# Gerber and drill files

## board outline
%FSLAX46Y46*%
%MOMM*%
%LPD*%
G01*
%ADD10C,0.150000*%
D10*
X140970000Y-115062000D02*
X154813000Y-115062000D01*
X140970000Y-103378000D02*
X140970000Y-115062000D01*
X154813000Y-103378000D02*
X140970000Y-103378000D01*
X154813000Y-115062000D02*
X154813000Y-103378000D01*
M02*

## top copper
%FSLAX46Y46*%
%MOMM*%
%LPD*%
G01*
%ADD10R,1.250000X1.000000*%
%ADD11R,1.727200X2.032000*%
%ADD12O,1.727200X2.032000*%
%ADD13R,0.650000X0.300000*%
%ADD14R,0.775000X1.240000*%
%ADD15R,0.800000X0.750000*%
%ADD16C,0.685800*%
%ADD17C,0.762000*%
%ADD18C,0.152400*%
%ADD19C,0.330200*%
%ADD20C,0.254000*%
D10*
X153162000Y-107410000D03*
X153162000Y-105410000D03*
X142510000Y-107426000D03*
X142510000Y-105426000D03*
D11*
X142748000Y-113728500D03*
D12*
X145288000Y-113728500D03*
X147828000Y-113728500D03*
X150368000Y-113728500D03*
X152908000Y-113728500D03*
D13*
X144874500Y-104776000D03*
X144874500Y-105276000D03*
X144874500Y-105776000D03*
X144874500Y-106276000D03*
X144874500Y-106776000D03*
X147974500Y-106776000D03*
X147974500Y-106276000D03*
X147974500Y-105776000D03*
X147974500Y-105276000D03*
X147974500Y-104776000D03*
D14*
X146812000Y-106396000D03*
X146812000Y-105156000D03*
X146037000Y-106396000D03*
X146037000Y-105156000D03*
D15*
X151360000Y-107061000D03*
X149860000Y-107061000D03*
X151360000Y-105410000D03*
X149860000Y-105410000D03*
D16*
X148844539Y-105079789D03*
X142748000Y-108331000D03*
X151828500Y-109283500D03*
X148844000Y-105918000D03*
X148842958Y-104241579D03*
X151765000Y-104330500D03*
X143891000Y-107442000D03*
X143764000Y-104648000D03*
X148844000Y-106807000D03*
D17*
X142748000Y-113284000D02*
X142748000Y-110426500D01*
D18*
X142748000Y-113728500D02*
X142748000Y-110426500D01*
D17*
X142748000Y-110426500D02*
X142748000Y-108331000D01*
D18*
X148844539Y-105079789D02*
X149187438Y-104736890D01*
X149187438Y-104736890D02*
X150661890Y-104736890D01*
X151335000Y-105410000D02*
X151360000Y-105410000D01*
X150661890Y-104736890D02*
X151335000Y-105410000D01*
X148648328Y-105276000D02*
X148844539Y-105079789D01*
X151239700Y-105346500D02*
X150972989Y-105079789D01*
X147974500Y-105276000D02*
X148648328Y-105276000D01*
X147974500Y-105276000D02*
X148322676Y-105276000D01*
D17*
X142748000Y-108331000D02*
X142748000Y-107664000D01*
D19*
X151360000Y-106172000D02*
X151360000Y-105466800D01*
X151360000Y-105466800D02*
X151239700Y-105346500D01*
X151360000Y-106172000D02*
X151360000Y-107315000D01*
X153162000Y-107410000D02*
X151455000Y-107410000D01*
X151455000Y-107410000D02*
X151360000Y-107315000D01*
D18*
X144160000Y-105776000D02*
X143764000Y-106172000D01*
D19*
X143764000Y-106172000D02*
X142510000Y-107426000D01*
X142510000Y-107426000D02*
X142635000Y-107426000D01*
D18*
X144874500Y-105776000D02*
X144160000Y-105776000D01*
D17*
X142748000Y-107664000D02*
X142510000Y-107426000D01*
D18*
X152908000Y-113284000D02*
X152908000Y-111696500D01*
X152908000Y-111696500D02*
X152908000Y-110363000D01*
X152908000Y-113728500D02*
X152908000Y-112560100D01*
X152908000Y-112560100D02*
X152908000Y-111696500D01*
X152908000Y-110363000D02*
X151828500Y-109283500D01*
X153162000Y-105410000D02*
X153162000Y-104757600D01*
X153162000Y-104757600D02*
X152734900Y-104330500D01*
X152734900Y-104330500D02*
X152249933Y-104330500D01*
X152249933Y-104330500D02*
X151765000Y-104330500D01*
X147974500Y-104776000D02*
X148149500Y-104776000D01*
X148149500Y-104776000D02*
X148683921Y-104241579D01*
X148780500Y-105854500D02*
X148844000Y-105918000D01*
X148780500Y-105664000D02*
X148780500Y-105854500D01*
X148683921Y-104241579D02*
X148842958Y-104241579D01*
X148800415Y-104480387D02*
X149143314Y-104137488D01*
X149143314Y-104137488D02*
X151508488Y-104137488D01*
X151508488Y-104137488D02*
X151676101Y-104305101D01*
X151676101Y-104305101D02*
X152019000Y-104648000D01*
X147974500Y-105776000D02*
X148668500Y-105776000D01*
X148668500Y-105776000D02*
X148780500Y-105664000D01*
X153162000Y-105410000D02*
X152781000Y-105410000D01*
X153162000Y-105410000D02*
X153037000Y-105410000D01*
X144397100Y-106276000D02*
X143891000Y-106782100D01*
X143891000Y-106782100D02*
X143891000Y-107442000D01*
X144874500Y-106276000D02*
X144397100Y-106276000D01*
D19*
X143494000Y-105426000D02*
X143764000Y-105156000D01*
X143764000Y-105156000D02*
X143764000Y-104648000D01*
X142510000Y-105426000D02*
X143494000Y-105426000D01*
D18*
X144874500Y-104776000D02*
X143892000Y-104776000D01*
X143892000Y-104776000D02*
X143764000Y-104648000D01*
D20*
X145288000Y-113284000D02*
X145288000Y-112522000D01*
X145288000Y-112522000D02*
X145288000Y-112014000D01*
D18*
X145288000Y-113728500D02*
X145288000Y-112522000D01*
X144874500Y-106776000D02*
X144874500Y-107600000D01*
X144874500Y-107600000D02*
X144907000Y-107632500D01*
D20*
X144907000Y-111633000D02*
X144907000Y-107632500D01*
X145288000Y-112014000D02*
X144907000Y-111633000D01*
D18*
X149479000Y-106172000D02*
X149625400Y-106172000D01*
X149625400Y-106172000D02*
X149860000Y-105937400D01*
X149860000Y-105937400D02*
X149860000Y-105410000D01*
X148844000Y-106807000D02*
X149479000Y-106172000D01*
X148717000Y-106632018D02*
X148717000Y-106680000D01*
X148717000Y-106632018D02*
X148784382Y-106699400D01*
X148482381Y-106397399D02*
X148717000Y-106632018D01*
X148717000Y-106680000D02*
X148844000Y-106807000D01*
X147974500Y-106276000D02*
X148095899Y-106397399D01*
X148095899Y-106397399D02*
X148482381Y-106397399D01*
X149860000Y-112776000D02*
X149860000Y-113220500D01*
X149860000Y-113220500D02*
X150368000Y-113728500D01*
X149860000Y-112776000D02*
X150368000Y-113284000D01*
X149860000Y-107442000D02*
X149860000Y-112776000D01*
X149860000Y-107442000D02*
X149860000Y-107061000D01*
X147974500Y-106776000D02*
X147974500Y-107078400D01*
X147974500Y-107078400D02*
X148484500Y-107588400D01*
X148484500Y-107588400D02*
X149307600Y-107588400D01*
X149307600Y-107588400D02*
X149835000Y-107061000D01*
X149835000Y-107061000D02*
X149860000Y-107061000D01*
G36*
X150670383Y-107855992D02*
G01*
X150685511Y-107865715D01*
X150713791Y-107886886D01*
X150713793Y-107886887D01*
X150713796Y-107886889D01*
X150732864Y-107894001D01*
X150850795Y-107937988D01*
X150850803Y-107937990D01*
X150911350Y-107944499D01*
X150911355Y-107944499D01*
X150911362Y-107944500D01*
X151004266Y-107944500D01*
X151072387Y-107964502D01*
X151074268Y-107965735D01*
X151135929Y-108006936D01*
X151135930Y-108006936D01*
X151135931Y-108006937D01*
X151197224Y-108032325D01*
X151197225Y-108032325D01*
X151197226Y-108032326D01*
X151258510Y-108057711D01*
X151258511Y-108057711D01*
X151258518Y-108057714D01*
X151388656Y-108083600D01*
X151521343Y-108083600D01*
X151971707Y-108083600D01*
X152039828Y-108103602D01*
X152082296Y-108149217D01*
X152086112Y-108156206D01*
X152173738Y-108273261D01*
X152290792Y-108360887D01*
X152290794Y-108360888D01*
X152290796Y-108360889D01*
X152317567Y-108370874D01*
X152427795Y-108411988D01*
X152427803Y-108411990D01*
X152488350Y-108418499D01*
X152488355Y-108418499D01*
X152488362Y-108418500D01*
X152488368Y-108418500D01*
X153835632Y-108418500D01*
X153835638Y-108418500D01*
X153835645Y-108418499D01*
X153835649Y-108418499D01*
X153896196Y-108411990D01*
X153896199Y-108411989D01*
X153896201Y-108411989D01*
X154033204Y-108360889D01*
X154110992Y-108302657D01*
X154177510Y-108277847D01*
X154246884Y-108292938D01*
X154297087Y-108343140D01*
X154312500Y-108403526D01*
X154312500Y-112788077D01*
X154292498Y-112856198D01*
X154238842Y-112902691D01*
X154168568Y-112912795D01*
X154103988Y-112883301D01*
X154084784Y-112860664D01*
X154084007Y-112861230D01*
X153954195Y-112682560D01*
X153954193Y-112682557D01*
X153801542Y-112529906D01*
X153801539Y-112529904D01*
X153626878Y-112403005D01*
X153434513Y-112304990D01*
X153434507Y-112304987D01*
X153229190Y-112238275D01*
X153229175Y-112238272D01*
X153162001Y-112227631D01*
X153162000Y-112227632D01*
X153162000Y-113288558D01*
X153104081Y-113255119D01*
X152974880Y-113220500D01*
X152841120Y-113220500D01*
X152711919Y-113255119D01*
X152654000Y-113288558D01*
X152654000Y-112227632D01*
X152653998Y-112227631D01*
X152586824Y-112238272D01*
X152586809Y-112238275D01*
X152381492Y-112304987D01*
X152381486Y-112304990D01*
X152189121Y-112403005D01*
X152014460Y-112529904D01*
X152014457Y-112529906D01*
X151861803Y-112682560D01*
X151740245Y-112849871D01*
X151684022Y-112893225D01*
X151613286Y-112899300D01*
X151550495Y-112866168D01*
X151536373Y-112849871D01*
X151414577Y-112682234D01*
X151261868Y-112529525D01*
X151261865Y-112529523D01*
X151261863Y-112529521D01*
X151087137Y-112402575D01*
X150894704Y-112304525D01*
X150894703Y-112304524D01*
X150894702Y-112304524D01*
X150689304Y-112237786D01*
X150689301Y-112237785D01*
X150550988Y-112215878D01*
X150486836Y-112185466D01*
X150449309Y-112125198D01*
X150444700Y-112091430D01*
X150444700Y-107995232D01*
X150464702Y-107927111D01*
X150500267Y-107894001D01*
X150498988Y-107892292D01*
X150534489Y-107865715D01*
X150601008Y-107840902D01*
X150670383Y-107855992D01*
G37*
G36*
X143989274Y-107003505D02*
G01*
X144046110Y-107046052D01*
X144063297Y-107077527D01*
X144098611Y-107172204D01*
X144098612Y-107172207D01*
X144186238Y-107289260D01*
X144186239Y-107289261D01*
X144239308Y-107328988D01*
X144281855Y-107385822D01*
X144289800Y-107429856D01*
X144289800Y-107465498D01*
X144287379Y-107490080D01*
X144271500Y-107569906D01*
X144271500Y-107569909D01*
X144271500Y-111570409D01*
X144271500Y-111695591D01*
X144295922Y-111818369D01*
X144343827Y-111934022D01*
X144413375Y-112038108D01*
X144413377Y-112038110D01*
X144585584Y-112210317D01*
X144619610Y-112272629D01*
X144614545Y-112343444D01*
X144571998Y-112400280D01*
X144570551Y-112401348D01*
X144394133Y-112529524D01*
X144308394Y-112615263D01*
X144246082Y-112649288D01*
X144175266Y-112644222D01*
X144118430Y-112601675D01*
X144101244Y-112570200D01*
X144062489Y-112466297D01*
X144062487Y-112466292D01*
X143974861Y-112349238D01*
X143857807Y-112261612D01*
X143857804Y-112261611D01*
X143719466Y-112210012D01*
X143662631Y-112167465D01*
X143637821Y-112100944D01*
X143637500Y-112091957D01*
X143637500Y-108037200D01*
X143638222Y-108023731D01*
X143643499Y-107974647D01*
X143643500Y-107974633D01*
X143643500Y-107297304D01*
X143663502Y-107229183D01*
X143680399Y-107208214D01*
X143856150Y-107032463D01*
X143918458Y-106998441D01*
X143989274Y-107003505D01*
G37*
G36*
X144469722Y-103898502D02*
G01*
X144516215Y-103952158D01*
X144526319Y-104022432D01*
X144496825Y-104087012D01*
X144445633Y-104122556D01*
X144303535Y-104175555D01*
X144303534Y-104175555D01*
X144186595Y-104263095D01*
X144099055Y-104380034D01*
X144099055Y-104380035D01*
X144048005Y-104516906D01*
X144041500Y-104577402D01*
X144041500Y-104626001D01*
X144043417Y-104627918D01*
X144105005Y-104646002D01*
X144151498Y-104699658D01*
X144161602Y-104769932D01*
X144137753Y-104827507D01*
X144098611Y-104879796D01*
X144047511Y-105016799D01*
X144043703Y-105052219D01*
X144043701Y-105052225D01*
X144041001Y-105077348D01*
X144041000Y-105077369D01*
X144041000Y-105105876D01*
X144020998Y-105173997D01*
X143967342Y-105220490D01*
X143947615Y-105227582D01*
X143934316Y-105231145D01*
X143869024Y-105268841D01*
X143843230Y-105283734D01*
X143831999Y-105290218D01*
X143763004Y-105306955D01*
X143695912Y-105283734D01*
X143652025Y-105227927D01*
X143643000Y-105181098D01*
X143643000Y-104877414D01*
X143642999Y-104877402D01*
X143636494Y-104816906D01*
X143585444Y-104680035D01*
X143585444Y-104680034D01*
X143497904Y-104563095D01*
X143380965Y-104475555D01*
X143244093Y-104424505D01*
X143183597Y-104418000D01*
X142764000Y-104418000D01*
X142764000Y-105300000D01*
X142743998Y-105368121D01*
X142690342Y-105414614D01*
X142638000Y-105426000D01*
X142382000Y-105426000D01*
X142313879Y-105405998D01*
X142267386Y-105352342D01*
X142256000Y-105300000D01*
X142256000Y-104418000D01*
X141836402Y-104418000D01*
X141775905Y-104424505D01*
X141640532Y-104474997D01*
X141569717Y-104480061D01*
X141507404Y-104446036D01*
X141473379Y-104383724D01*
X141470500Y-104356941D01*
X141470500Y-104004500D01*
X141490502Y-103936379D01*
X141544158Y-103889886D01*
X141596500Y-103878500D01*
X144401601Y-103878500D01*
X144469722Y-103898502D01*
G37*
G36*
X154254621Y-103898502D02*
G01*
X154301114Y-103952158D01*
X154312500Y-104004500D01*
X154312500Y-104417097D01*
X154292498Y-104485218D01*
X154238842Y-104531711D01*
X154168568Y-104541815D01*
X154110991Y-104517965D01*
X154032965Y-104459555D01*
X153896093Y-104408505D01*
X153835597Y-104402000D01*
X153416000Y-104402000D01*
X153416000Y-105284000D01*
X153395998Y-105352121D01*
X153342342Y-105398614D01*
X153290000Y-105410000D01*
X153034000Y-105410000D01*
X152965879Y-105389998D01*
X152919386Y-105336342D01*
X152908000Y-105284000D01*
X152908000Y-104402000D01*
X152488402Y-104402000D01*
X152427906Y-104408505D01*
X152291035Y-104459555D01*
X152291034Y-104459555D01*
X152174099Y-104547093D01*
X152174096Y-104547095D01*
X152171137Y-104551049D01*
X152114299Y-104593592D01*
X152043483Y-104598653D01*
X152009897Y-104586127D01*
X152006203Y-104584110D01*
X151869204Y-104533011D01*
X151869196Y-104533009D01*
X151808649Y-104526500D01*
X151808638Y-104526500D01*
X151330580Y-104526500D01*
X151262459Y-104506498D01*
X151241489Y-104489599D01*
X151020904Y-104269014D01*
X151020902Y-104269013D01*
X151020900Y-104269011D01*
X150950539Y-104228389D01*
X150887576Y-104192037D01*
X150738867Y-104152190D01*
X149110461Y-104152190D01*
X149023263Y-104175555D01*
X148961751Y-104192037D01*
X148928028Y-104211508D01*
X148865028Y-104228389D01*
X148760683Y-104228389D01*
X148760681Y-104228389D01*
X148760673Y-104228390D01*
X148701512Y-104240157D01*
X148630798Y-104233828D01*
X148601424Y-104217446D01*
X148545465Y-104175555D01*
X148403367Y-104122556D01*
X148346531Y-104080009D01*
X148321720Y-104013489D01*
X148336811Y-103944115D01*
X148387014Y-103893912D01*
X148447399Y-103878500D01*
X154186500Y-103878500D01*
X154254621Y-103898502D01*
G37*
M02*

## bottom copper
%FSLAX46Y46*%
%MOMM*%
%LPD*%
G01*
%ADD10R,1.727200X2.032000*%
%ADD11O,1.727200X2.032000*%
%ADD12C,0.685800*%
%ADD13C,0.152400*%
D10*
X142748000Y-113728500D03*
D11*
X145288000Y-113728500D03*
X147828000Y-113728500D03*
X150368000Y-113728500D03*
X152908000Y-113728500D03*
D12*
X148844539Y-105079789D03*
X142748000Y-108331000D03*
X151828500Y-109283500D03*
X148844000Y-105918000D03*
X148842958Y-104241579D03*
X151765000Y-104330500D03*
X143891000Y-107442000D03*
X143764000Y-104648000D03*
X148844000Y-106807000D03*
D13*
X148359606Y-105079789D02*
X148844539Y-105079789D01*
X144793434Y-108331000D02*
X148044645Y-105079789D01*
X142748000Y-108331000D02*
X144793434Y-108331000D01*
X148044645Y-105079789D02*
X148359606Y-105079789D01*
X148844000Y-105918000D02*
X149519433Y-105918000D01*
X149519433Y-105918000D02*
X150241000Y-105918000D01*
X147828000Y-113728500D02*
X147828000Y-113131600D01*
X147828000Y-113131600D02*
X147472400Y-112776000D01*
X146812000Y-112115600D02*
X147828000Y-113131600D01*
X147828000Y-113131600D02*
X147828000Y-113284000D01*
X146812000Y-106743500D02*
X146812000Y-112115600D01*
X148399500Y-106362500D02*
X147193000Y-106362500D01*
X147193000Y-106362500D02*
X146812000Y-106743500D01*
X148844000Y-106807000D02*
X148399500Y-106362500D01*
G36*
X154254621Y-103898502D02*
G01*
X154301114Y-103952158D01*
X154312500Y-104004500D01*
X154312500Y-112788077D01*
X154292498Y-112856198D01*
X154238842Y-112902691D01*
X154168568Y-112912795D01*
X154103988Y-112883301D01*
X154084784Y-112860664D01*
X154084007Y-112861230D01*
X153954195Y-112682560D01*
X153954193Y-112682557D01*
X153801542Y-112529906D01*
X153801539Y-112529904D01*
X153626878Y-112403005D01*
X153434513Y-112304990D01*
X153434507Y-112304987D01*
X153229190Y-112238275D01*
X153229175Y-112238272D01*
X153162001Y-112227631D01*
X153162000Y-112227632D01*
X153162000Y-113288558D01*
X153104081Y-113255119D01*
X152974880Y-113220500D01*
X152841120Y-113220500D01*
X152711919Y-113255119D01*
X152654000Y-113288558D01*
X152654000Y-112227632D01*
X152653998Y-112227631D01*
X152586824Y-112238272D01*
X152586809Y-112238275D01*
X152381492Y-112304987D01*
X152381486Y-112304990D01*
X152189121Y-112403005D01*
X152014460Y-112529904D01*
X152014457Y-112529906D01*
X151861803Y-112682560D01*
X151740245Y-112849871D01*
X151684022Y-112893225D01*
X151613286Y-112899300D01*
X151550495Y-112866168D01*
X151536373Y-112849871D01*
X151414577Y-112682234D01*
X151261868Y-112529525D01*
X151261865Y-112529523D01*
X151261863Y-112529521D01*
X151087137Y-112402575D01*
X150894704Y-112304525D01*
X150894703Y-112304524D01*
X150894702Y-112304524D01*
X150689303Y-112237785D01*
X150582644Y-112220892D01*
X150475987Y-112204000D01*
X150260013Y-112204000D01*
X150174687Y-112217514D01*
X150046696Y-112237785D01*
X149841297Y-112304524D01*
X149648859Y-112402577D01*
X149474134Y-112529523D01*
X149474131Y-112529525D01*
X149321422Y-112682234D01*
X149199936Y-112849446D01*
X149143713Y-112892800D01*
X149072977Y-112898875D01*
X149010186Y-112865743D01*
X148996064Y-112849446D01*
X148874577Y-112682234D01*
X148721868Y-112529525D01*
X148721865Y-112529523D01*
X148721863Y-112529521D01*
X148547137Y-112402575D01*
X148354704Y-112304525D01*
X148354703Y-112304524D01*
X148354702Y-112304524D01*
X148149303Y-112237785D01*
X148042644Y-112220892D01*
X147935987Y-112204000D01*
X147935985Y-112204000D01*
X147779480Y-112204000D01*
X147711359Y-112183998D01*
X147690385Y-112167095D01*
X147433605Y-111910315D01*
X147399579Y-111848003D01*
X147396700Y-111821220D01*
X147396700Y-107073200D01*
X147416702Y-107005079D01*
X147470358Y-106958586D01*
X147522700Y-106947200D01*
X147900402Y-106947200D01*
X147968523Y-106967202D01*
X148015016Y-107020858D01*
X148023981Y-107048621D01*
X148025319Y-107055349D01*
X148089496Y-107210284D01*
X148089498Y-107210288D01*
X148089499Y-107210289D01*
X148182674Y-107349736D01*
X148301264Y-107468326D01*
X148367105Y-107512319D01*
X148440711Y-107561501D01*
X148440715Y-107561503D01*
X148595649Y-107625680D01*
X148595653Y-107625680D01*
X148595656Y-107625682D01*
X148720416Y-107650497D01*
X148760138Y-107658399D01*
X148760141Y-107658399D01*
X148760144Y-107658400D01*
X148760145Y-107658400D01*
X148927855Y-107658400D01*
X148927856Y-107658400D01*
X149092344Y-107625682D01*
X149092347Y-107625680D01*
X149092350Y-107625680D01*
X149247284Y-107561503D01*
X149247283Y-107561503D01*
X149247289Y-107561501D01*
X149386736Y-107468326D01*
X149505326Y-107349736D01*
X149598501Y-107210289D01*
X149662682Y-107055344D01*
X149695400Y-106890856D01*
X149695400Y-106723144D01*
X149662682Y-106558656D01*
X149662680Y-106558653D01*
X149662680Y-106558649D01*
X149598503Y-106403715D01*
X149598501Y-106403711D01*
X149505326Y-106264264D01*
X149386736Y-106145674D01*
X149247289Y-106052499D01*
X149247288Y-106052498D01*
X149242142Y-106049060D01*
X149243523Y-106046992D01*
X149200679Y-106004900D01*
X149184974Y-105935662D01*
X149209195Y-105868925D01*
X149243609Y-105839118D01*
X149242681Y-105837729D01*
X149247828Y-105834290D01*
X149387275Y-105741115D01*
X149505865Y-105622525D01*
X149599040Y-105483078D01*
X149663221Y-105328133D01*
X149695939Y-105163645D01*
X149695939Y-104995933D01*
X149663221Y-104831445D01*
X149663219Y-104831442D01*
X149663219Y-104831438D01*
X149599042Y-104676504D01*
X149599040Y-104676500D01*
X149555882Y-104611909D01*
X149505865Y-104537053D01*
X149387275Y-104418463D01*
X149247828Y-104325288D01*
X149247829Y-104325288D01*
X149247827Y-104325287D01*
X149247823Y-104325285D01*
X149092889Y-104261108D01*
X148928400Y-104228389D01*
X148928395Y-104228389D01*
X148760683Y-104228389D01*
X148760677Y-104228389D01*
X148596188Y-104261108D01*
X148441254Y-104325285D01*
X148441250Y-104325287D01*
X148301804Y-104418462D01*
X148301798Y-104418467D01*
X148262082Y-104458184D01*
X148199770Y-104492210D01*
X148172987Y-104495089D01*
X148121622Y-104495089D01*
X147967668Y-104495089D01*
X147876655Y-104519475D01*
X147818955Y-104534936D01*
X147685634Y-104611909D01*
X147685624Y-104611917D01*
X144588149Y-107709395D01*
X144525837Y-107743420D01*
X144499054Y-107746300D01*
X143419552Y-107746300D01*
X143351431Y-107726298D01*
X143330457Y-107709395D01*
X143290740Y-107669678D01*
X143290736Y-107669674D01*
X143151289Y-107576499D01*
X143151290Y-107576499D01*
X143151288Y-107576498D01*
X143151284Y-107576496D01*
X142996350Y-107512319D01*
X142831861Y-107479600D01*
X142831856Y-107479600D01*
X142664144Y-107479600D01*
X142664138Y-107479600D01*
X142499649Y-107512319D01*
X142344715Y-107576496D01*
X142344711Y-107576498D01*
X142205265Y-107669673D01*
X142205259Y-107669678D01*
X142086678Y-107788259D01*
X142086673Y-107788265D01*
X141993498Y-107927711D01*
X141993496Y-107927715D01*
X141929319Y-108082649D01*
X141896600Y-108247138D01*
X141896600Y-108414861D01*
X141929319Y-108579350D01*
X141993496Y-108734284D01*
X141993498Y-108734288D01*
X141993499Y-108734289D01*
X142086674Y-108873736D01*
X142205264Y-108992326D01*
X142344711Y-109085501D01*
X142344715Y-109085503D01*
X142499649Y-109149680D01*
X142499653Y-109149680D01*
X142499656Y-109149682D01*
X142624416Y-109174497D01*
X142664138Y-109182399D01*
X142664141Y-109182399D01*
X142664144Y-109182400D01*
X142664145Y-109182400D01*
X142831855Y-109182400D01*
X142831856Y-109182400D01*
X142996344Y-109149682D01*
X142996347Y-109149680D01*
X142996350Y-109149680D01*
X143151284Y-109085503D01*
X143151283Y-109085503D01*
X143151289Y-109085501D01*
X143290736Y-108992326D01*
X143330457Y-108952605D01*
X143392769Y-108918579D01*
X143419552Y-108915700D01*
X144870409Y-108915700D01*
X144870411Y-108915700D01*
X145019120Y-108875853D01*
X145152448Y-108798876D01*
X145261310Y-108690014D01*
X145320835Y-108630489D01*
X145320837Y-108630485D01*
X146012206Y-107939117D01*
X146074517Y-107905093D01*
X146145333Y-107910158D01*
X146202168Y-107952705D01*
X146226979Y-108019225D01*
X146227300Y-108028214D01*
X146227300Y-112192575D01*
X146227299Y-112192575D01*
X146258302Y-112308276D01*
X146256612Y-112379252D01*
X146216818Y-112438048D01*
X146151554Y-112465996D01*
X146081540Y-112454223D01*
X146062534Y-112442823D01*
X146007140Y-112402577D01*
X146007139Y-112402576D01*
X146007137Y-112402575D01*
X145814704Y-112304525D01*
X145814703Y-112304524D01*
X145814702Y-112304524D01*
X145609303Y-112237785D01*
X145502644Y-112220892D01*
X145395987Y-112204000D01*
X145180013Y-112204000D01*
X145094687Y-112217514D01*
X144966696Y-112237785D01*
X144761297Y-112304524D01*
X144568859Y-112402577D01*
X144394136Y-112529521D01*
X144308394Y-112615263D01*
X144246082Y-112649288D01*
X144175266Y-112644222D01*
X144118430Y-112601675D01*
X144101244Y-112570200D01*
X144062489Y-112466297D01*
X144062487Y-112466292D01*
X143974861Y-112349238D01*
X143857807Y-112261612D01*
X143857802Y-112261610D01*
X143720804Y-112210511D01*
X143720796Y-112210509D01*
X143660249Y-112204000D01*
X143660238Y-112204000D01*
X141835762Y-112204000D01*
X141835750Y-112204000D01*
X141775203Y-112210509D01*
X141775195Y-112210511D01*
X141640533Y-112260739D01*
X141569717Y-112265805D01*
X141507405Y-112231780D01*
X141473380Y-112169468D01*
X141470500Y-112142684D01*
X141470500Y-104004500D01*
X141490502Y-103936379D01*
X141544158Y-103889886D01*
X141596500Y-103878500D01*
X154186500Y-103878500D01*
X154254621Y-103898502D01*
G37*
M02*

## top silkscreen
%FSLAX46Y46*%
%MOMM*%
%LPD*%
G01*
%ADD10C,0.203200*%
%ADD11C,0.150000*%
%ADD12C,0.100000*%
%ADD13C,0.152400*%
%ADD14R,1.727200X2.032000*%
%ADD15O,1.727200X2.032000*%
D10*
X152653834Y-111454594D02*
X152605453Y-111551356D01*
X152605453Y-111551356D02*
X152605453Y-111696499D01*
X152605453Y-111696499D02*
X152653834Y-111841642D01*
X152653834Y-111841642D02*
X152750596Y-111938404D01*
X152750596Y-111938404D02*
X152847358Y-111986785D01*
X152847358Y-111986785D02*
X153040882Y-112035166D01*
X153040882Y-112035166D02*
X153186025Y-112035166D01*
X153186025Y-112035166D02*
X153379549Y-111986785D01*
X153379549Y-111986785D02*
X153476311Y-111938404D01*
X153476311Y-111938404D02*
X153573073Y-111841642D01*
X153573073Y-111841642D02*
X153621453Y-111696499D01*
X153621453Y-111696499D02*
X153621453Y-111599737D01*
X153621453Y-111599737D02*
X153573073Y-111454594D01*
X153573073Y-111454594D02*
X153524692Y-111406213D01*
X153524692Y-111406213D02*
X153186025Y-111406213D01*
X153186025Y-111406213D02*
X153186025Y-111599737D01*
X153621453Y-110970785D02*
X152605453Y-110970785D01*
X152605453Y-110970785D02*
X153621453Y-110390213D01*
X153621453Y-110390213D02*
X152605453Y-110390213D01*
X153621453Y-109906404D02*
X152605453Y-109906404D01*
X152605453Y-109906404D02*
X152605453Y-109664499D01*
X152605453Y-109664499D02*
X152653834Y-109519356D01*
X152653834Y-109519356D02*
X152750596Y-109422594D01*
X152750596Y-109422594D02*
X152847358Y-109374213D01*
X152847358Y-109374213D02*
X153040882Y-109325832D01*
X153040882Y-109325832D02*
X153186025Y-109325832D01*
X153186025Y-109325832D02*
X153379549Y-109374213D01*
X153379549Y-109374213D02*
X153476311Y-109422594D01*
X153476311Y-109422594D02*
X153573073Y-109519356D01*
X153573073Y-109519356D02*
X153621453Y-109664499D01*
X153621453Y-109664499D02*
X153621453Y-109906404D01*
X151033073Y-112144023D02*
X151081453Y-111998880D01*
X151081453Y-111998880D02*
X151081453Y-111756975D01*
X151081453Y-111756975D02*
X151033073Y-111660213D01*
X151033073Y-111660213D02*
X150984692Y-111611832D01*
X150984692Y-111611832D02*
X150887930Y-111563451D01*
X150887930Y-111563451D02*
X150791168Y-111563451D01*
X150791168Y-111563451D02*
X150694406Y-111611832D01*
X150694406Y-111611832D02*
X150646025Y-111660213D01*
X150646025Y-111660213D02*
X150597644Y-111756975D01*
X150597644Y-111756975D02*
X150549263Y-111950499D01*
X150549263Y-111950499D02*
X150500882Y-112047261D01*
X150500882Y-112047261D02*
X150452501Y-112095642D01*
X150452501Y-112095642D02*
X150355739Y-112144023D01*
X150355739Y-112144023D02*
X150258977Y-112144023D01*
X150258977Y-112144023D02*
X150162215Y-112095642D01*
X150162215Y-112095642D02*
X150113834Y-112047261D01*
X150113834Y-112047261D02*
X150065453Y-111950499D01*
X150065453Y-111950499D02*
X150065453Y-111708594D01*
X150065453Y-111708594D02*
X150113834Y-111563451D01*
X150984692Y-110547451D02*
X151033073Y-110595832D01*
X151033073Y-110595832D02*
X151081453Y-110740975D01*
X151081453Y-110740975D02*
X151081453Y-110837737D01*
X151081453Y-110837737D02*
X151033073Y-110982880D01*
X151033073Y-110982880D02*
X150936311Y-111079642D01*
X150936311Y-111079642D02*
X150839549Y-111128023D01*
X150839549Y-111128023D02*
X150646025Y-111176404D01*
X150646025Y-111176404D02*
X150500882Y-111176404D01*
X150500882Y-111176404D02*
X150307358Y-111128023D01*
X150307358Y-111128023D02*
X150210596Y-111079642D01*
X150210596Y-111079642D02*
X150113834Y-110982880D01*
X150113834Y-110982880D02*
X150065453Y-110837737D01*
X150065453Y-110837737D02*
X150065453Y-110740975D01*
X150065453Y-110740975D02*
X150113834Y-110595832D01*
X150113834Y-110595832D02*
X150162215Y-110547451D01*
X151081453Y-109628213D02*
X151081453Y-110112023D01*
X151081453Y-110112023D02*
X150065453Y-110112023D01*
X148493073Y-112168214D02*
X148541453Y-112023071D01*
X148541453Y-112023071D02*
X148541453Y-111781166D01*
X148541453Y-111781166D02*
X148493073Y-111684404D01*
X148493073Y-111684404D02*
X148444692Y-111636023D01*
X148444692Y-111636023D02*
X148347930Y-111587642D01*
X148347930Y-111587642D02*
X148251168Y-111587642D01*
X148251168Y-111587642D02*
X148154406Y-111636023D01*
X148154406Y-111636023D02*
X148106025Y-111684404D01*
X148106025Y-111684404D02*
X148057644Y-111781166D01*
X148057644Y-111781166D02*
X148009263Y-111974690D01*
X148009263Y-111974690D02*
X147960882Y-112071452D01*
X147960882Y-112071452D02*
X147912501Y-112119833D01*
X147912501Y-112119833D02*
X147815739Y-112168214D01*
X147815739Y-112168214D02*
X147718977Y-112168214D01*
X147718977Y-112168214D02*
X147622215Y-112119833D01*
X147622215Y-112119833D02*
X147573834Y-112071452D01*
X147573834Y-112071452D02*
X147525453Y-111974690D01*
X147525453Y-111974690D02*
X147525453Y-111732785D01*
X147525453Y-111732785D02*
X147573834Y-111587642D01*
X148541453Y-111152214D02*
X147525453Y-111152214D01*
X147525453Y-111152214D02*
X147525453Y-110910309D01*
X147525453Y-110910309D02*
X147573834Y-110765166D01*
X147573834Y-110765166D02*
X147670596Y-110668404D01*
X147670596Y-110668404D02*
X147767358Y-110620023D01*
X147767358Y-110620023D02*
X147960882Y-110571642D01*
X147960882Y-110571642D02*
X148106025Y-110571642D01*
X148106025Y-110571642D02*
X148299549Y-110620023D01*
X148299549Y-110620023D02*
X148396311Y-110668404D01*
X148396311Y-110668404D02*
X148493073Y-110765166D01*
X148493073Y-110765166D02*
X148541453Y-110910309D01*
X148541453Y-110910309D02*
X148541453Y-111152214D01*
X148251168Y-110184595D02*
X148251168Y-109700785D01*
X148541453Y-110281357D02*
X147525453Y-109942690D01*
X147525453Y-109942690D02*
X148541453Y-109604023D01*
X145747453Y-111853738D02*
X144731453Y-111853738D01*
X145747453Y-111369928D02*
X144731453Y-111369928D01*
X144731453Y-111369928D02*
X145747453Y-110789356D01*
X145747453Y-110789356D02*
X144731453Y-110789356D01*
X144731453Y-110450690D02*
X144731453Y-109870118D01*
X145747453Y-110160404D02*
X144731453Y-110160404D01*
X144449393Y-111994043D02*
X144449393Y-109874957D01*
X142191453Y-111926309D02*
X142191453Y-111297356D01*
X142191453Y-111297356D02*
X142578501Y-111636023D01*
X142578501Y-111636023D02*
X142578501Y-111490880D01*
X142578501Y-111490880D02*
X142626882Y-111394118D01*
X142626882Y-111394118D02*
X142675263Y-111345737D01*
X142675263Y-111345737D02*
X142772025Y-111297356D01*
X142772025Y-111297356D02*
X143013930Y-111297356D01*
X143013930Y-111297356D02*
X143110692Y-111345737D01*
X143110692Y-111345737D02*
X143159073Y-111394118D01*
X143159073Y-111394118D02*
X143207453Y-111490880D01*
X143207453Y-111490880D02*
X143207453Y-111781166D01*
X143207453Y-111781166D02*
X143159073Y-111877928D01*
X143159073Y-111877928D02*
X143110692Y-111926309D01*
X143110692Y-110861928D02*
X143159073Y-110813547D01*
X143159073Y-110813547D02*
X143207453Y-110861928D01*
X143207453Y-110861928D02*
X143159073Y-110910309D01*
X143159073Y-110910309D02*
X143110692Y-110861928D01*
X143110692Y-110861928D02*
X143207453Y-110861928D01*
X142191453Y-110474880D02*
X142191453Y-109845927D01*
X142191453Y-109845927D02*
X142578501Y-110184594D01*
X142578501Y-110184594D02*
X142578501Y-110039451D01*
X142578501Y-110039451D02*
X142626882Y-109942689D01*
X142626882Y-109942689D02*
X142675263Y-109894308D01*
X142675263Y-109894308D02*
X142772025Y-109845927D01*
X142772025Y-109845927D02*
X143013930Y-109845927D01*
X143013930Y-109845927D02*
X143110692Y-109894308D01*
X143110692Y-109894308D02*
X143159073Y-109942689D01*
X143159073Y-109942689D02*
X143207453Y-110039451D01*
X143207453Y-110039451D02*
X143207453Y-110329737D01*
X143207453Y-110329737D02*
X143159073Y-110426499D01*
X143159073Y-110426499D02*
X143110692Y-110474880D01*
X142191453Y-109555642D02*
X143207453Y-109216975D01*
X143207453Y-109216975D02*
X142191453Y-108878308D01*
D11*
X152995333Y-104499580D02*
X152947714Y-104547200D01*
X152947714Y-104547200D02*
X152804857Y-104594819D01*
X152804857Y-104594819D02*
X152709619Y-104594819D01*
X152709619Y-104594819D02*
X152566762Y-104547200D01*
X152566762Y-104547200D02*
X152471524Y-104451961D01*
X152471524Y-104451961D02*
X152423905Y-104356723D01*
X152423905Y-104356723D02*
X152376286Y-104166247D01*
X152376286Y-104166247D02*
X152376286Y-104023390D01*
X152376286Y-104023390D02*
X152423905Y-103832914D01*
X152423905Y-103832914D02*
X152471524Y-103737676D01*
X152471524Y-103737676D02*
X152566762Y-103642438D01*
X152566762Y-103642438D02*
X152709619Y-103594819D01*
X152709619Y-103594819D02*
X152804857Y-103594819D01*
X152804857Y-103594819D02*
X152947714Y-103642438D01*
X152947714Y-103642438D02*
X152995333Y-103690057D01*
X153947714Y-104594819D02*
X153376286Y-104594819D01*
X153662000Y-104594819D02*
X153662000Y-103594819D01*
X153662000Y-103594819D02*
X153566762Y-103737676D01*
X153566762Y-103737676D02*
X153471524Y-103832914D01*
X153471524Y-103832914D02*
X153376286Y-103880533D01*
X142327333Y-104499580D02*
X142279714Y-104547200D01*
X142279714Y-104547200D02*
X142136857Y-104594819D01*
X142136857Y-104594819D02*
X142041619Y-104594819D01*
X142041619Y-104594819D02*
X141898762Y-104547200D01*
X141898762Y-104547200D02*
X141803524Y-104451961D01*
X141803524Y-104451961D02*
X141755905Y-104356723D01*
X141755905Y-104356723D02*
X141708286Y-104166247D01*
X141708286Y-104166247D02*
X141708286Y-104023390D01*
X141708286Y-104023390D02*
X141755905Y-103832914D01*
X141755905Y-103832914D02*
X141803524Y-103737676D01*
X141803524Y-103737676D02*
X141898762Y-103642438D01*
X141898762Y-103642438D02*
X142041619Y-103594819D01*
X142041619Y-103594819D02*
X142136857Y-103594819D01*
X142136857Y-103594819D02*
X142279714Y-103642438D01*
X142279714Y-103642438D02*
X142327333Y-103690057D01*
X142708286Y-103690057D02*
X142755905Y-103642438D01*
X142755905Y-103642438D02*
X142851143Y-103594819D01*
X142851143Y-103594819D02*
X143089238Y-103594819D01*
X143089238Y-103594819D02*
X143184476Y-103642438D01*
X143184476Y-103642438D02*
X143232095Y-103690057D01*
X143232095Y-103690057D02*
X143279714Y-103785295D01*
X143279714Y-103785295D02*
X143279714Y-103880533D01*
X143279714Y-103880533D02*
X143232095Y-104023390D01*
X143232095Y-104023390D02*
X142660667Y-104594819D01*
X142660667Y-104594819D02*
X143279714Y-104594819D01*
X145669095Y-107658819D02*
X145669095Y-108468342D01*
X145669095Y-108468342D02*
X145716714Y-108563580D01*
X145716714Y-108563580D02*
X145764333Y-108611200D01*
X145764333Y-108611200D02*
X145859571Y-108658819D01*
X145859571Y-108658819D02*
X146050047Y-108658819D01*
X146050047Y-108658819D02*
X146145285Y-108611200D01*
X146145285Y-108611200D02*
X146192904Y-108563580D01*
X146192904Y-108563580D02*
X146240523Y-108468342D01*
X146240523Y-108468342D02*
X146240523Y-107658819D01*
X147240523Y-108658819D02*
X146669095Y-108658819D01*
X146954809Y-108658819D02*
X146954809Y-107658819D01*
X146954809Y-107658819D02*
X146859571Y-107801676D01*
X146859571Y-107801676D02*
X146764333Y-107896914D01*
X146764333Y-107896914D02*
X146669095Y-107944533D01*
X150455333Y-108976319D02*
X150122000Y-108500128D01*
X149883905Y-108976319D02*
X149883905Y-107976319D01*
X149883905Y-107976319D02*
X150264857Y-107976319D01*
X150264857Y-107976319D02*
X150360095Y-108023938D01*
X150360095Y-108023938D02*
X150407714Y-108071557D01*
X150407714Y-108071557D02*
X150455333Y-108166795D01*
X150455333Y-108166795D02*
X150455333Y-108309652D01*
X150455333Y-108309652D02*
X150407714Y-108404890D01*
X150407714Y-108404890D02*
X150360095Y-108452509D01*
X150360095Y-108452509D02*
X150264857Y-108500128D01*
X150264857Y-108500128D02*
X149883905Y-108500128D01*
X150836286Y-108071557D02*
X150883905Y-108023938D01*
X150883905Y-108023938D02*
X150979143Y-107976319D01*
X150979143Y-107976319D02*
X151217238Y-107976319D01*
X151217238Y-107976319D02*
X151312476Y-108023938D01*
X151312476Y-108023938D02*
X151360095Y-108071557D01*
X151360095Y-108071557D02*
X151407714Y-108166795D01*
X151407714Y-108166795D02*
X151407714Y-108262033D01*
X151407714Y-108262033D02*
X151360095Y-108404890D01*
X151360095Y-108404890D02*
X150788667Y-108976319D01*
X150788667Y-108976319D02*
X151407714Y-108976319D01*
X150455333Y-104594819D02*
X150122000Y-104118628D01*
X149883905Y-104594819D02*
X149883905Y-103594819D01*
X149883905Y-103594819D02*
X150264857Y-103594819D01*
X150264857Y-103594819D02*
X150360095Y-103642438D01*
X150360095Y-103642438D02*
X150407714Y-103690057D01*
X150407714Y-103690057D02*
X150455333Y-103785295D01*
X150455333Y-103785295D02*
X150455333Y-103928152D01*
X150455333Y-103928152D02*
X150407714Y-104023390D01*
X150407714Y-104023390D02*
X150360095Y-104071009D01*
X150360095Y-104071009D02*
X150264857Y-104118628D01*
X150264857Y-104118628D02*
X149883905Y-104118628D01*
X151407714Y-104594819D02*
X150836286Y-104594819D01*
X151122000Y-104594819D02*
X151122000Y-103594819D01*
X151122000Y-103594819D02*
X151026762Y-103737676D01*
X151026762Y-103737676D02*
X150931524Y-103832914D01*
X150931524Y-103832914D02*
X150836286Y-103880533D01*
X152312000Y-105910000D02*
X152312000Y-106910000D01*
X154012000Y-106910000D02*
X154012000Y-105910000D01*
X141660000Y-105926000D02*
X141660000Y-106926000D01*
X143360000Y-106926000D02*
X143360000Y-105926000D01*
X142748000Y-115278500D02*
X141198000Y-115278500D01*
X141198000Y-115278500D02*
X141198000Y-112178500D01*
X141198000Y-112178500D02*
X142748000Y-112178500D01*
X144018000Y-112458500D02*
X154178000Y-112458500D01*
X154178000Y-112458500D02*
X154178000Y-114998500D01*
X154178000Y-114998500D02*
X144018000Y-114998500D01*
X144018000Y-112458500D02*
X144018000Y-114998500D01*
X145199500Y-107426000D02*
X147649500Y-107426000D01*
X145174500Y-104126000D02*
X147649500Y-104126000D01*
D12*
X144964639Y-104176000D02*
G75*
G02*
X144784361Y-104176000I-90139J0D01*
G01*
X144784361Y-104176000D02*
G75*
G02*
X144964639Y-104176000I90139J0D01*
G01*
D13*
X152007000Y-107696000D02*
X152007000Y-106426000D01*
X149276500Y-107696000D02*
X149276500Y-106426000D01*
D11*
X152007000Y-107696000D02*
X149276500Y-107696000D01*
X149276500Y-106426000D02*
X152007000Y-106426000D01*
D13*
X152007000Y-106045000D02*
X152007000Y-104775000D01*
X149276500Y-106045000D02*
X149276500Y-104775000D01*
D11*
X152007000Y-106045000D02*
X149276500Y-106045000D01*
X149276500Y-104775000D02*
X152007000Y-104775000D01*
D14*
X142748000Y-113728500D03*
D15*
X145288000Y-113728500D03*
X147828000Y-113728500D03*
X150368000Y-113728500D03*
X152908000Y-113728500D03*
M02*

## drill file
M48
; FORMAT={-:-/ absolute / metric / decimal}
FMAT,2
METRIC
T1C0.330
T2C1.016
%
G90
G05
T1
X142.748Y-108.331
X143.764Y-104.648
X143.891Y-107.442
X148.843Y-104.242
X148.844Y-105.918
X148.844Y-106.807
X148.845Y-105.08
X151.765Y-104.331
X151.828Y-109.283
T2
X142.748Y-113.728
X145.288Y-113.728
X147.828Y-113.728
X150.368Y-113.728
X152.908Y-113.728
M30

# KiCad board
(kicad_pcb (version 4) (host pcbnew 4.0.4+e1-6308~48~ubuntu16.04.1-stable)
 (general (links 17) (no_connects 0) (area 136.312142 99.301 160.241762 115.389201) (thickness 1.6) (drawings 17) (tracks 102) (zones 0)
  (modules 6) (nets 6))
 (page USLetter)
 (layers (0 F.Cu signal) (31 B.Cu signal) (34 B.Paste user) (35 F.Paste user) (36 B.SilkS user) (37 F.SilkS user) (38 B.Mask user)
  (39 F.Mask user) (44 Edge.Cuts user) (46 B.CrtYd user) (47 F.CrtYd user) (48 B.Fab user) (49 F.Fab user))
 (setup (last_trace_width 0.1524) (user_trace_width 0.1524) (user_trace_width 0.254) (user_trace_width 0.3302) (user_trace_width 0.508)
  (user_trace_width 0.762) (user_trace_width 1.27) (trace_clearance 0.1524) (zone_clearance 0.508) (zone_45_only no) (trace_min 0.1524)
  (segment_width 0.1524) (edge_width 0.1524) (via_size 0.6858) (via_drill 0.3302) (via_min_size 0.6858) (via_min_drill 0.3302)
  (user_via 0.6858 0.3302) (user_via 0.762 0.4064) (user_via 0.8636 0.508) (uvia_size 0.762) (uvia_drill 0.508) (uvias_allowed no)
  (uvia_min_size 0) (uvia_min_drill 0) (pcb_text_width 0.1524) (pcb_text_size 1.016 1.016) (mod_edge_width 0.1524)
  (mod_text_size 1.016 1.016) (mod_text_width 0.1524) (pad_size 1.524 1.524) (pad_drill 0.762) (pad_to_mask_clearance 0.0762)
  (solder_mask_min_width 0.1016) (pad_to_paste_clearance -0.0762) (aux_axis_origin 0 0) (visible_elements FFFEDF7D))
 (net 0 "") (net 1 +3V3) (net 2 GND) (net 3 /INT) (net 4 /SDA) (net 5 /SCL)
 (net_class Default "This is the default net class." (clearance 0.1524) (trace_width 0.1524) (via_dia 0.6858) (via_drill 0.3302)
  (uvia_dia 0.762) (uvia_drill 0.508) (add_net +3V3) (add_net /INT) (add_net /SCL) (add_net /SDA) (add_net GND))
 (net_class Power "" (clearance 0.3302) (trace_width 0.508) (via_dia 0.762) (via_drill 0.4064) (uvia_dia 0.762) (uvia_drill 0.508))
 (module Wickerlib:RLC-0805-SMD (layer F.Cu) (at 153.162 106.41 90)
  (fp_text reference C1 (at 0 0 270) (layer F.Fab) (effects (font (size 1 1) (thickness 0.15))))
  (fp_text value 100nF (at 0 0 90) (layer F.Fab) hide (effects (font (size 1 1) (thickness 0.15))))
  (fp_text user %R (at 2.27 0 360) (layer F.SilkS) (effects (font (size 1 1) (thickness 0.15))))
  (fp_line (start 0.5 -0.85) (end -0.5 -0.85) (layer F.SilkS) (width 0.15))
  (fp_line (start -0.5 0.85) (end 0.5 0.85) (layer F.SilkS) (width 0.15))
  (pad 1 smd rect (at -1 0 90) (size 1 1.25) (layers F.Cu F.Paste F.Mask) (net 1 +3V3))
  (pad 2 smd rect (at 1 0 90) (size 1 1.25) (layers F.Cu F.Paste F.Mask) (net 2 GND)))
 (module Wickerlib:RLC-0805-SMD (layer F.Cu) (at 142.51 106.426 90)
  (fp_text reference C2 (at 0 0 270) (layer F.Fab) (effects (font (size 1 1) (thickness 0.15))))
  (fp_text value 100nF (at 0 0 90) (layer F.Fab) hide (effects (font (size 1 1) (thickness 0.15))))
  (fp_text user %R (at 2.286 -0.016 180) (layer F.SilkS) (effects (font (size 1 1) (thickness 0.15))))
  (fp_line (start 0.5 -0.85) (end -0.5 -0.85) (layer F.SilkS) (width 0.15))
  (fp_line (start -0.5 0.85) (end 0.5 0.85) (layer F.SilkS) (width 0.15))
  (pad 1 smd rect (at -1 0 90) (size 1 1.25) (layers F.Cu F.Paste F.Mask) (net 1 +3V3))
  (pad 2 smd rect (at 1 0 90) (size 1 1.25) (layers F.Cu F.Paste F.Mask) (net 2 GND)))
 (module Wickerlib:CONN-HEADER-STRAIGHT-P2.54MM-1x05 (layer F.Cu) (at 142.748 113.7285 90)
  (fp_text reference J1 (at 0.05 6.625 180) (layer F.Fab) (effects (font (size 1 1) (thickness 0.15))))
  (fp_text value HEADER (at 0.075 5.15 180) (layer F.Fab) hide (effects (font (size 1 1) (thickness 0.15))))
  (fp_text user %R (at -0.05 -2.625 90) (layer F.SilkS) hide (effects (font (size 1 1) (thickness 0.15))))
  (fp_line (start -1.55 0) (end -1.55 -1.55) (layer F.SilkS) (width 0.15))
  (fp_line (start -1.55 -1.55) (end 1.55 -1.55) (layer F.SilkS) (width 0.15))
  (fp_line (start 1.55 -1.55) (end 1.55 0) (layer F.SilkS) (width 0.15))
  (fp_line (start 1.27 1.27) (end 1.27 11.43) (layer F.SilkS) (width 0.15))
  (fp_line (start 1.27 11.43) (end -1.27 11.43) (layer F.SilkS) (width 0.15))
  (fp_line (start -1.27 11.43) (end -1.27 1.27) (layer F.SilkS) (width 0.15))
  (fp_line (start 1.27 1.27) (end -1.27 1.27) (layer F.SilkS) (width 0.15))
  (pad 1 thru_hole rect (at 0 0 90) (size 2.032 1.7272) (drill 1.016) (layers *.Cu *.Mask F.SilkS) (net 1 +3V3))
  (pad 2 thru_hole oval (at 0 2.54 90) (size 2.032 1.7272) (drill 1.016) (layers *.Cu *.Mask F.SilkS) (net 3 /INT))
  (pad 3 thru_hole oval (at 0 5.08 90) (size 2.032 1.7272) (drill 1.016) (layers *.Cu *.Mask F.SilkS) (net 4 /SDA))
  (pad 4 thru_hole oval (at 0 7.62 90) (size 2.032 1.7272) (drill 1.016) (layers *.Cu *.Mask F.SilkS) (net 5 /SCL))
  (pad 5 thru_hole oval (at 0 10.16 90) (size 2.032 1.7272) (drill 1.016) (layers *.Cu *.Mask F.SilkS) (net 2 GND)))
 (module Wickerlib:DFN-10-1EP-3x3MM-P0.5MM (layer F.Cu) (at 146.4245 105.776)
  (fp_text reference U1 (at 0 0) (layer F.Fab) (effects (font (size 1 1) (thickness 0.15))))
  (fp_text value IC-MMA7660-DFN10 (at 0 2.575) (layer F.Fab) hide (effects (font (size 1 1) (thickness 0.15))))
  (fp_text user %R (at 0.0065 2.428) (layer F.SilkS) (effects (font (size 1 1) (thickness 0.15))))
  (fp_line (start -1.225 1.65) (end 1.225 1.65) (layer F.SilkS) (width 0.15))
  (fp_line (start -1.25 -1.65) (end 1.225 -1.65) (layer F.SilkS) (width 0.15))
  (fp_circle (center -1.55 -1.6) (end -1.5 -1.525) (layer F.SilkS) (width 0.1))
  (pad 1 smd rect (at -1.55 -1) (size 0.65 0.3) (layers F.Cu F.Paste F.Mask) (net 2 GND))
  (pad 2 smd rect (at -1.55 -0.5) (size 0.65 0.3) (layers F.Cu F.Paste F.Mask))
  (pad 3 smd rect (at -1.55 0) (size 0.65 0.3) (layers F.Cu F.Paste F.Mask) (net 1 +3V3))
  (pad 4 smd rect (at -1.55 0.5) (size 0.65 0.3) (layers F.Cu F.Paste F.Mask) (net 2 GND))
  (pad 5 smd rect (at -1.55 1) (size 0.65 0.3) (layers F.Cu F.Paste F.Mask) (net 3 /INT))
  (pad 6 smd rect (at 1.55 1) (size 0.65 0.3) (layers F.Cu F.Paste F.Mask) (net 5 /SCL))
  (pad 7 smd rect (at 1.55 0.5) (size 0.65 0.3) (layers F.Cu F.Paste F.Mask) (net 4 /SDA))
  (pad 8 smd rect (at 1.55 0) (size 0.65 0.3) (layers F.Cu F.Paste F.Mask) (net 2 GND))
  (pad 9 smd rect (at 1.55 -0.5) (size 0.65 0.3) (layers F.Cu F.Paste F.Mask) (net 1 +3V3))
  (pad 10 smd rect (at 1.55 -1) (size 0.65 0.3) (layers F.Cu F.Paste F.Mask) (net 2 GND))
  (pad 11 smd rect (at 0.3875 0.62) (size 0.775 1.24) (layers F.Cu F.Paste F.Mask) (solder_paste_margin_ratio -0.2))
  (pad 11 smd rect (at 0.3875 -0.62) (size 0.775 1.24) (layers F.Cu F.Paste F.Mask) (solder_paste_margin_ratio -0.2))
  (pad 11 smd rect (at -0.3875 0.62) (size 0.775 1.24) (layers F.Cu F.Paste F.Mask) (solder_paste_margin_ratio -0.2))
  (pad 11 smd rect (at -0.3875 -0.62) (size 0.775 1.24) (layers F.Cu F.Paste F.Mask) (solder_paste_margin_ratio -0.2)))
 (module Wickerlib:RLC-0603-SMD (layer F.Cu) (at 150.61 107.061 180)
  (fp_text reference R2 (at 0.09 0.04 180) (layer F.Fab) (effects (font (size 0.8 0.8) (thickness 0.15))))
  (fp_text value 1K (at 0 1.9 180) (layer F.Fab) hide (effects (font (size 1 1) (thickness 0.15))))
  (fp_line (start -1.397 -0.635) (end -1.397 0.635) (layer F.SilkS) (width 0.1524))
  (fp_line (start 1.3335 -0.635) (end 1.3335 0.635) (layer F.SilkS) (width 0.1524))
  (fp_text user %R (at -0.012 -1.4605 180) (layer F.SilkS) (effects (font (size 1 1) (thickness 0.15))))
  (fp_line (start -1.397 -0.635) (end 1.3335 -0.635) (layer F.SilkS) (width 0.15))
  (fp_line (start 1.3335 0.635) (end -1.397 0.635) (layer F.SilkS) (width 0.15))
  (pad 1 smd rect (at -0.75 0 180) (size 0.8 0.75) (layers F.Cu F.Paste F.Mask) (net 1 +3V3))
  (pad 2 smd rect (at 0.75 0 180) (size 0.8 0.75) (layers F.Cu F.Paste F.Mask) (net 5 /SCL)))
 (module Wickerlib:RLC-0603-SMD (layer F.Cu) (at 150.61 105.41 180)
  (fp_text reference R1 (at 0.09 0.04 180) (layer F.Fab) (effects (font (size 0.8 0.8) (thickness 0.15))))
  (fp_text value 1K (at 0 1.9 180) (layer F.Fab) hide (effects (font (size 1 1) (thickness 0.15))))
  (fp_line (start -1.397 -0.635) (end -1.397 0.635) (layer F.SilkS) (width 0.1524))
  (fp_line (start 1.3335 -0.635) (end 1.3335 0.635) (layer F.SilkS) (width 0.1524))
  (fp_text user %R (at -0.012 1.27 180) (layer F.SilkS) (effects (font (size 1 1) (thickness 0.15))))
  (fp_line (start -1.397 -0.635) (end 1.3335 -0.635) (layer F.SilkS) (width 0.15))
  (fp_line (start 1.3335 0.635) (end -1.397 0.635) (layer F.SilkS) (width 0.15))
  (pad 1 smd rect (at -0.75 0 180) (size 0.8 0.75) (layers F.Cu F.Paste F.Mask) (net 1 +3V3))
  (pad 2 smd rect (at 0.75 0 180) (size 0.8 0.75) (layers F.Cu F.Paste F.Mask) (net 4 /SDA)))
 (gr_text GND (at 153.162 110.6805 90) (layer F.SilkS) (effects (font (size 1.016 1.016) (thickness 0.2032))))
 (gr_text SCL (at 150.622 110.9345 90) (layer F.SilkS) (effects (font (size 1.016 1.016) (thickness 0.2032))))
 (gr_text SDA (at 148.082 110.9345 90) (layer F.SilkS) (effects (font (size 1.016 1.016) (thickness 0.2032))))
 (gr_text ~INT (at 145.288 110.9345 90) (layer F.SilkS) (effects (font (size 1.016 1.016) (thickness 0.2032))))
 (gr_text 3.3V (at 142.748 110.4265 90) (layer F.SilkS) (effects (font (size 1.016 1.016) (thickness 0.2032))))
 (gr_line (start 140.97 115.062) (end 154.813 115.062) (layer Edge.Cuts) (width 0.15))
 (gr_line (start 140.97 103.378) (end 140.97 115.062) (layer Edge.Cuts) (width 0.15))
 (gr_line (start 154.813 103.378) (end 140.97 103.378) (layer Edge.Cuts) (width 0.15))
 (gr_line (start 154.813 115.062) (end 154.813 103.378) (layer Edge.Cuts) (width 0.15))
 (segment (start 142.748 113.284) (end 142.748 110.4265) (width 0.762) (layer F.Cu) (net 1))
 (segment (start 142.748 113.7285) (end 142.748 110.4265) (width 0.1524) (layer F.Cu) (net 1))
 (segment (start 142.748 110.4265) (end 142.748 108.331) (width 0.762) (layer F.Cu) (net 1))
 (segment (start 148.844539 105.079789) (end 149.187438 104.73689) (width 0.1524) (layer F.Cu) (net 1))
 (segment (start 149.187438 104.73689) (end 150.66189 104.73689) (width 0.1524) (layer F.Cu) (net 1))
 (segment (start 151.335 105.41) (end 151.36 105.41) (width 0.1524) (layer F.Cu) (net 1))
 (segment (start 150.66189 104.73689) (end 151.335 105.41) (width 0.1524) (layer F.Cu) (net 1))
 (segment (start 148.359606 105.079789) (end 148.844539 105.079789) (width 0.1524) (layer B.Cu) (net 1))
 (segment (start 144.793434 108.331) (end 148.044645 105.079789) (width 0.1524) (layer B.Cu) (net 1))
 (segment (start 142.748 108.331) (end 144.793434 108.331) (width 0.1524) (layer B.Cu) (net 1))
 (segment (start 148.044645 105.079789) (end 148.359606 105.079789) (width 0.1524) (layer B.Cu) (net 1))
 (segment (start 148.648328 105.276) (end 148.844539 105.079789) (width 0.1524) (layer F.Cu) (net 1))
 (segment (start 151.2397 105.3465) (end 150.972989 105.079789) (width 0.1524) (layer F.Cu) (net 1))
 (segment (start 147.9745 105.276) (end 148.648328 105.276) (width 0.1524) (layer F.Cu) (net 1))
 (via (at 148.844539 105.079789) (size 0.6858) (drill 0.3302) (layers F.Cu B.Cu) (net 1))
 (segment (start 147.9745 105.276) (end 148.322676 105.276) (width 0.1524) (layer F.Cu) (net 1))
 (segment (start 142.748 108.331) (end 142.748 107.664) (width 0.762) (layer F.Cu) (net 1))
 (via (at 142.748 108.331) (size 0.6858) (drill 0.3302) (layers F.Cu B.Cu) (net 1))
 (segment (start 151.36 106.172) (end 151.36 105.4668) (width 0.3302) (layer F.Cu) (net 1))
 (segment (start 151.36 105.4668) (end 151.2397 105.3465) (width 0.3302) (layer F.Cu) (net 1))
 (segment (start 151.36 106.172) (end 151.36 107.315) (width 0.3302) (layer F.Cu) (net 1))
 (segment (start 153.162 107.41) (end 151.455 107.41) (width 0.3302) (layer F.Cu) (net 1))
 (segment (start 151.455 107.41) (end 151.36 107.315) (width 0.3302) (layer F.Cu) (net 1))
 (segment (start 144.16 105.776) (end 143.764 106.172) (width 0.1524) (layer F.Cu) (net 1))
 (segment (start 143.764 106.172) (end 142.51 107.426) (width 0.3302) (layer F.Cu) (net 1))
 (segment (start 142.51 107.426) (end 142.635 107.426) (width 0.3302) (layer F.Cu) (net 1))
 (segment (start 144.8745 105.776) (end 144.16 105.776) (width 0.1524) (layer F.Cu) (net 1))
 (segment (start 142.748 107.664) (end 142.51 107.426) (width 0.762) (layer F.Cu) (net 1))
 (segment (start 152.908 113.284) (end 152.908 111.6965) (width 0.1524) (layer F.Cu) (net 2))
 (segment (start 152.908 111.6965) (end 152.908 110.363) (width 0.1524) (layer F.Cu) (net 2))
 (segment (start 152.908 113.7285) (end 152.908 112.5601) (width 0.1524) (layer F.Cu) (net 2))
 (segment (start 152.908 112.5601) (end 152.908 111.6965) (width 0.1524) (layer F.Cu) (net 2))
 (segment (start 152.908 110.363) (end 151.8285 109.2835) (width 0.1524) (layer F.Cu) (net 2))
 (via (at 151.8285 109.2835) (size 0.6858) (drill 0.3302) (layers F.Cu B.Cu) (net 2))
 (segment (start 153.162 105.41) (end 153.162 104.7576) (width 0.1524) (layer F.Cu) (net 2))
 (segment (start 153.162 104.7576) (end 152.7349 104.3305) (width 0.1524) (layer F.Cu) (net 2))
 (segment (start 152.7349 104.3305) (end 152.249933 104.3305) (width 0.1524) (layer F.Cu) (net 2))
 (segment (start 152.249933 104.3305) (end 151.765 104.3305) (width 0.1524) (layer F.Cu) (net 2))
 (segment (start 148.844 105.918) (end 149.519433 105.918) (width 0.1524) (layer B.Cu) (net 2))
 (segment (start 147.9745 104.776) (end 148.1495 104.776) (width 0.1524) (layer F.Cu) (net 2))
 (via (at 148.844 105.918) (size 0.6858) (drill 0.3302) (layers F.Cu B.Cu) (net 2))
 (segment (start 148.1495 104.776) (end 148.683921 104.241579) (width 0.1524) (layer F.Cu) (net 2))
 (segment (start 148.7805 105.8545) (end 148.844 105.918) (width 0.1524) (layer F.Cu) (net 2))
 (segment (start 148.7805 105.664) (end 148.7805 105.8545) (width 0.1524) (layer F.Cu) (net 2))
 (via (at 148.842958 104.241579) (size 0.6858) (drill 0.3302) (layers F.Cu B.Cu) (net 2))
 (segment (start 148.683921 104.241579) (end 148.842958 104.241579) (width 0.1524) (layer F.Cu) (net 2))
 (segment (start 148.800415 104.480387) (end 149.143314 104.137488) (width 0.1524) (layer F.Cu) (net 2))
 (segment (start 149.143314 104.137488) (end 151.508488 104.137488) (width 0.1524) (layer F.Cu) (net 2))
 (segment (start 151.508488 104.137488) (end 151.676101 104.305101) (width 0.1524) (layer F.Cu) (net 2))
 (segment (start 151.676101 104.305101) (end 152.019 104.648) (width 0.1524) (layer F.Cu) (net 2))
 (segment (start 149.519433 105.918) (end 150.241 105.918) (width 0.1524) (layer B.Cu) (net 2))
 (segment (start 147.9745 105.776) (end 148.6685 105.776) (width 0.1524) (layer F.Cu) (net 2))
 (segment (start 148.6685 105.776) (end 148.7805 105.664) (width 0.1524) (layer F.Cu) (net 2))
 (segment (start 153.162 105.41) (end 152.781 105.41) (width 0.1524) (layer F.Cu) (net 2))
 (via (at 151.765 104.3305) (size 0.6858) (drill 0.3302) (layers F.Cu B.Cu) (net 2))
 (segment (start 153.162 105.41) (end 153.037 105.41) (width 0.1524) (layer F.Cu) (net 2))
 (segment (start 144.3971 106.276) (end 143.891 106.7821) (width 0.1524) (layer F.Cu) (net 2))
 (segment (start 143.891 106.7821) (end 143.891 107.442) (width 0.1524) (layer F.Cu) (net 2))
 (segment (start 144.8745 106.276) (end 144.3971 106.276) (width 0.1524) (layer F.Cu) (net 2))
 (via (at 143.891 107.442) (size 0.6858) (drill 0.3302) (layers F.Cu B.Cu) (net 2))
 (segment (start 143.494 105.426) (end 143.764 105.156) (width 0.3302) (layer F.Cu) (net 2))
 (segment (start 143.764 105.156) (end 143.764 104.648) (width 0.3302) (layer F.Cu) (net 2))
 (segment (start 142.51 105.426) (end 143.494 105.426) (width 0.3302) (layer F.Cu) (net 2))
 (segment (start 144.8745 104.776) (end 143.892 104.776) (width 0.1524) (layer F.Cu) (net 2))
 (segment (start 143.892 104.776) (end 143.764 104.648) (width 0.1524) (layer F.Cu) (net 2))
 (via (at 143.764 104.648) (size 0.6858) (drill 0.3302) (layers F.Cu B.Cu) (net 2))
 (segment (start 145.288 113.284) (end 145.288 112.522) (width 0.254) (layer F.Cu) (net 3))
 (segment (start 145.288 112.522) (end 145.288 112.014) (width 0.254) (layer F.Cu) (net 3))
 (segment (start 145.288 113.7285) (end 145.288 112.522) (width 0.1524) (layer F.Cu) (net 3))
 (segment (start 144.8745 106.776) (end 144.8745 107.6) (width 0.1524) (layer F.Cu) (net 3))
 (segment (start 144.8745 107.6) (end 144.907 107.6325) (width 0.1524) (layer F.Cu) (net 3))
 (segment (start 144.907 111.633) (end 144.907 107.6325) (width 0.254) (layer F.Cu) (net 3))
 (segment (start 145.288 112.014) (end 144.907 111.633) (width 0.254) (layer F.Cu) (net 3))
 (segment (start 147.828 113.7285) (end 147.828 113.1316) (width 0.1524) (layer B.Cu) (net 4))
 (segment (start 147.828 113.1316) (end 147.4724 112.776) (width 0.1524) (layer B.Cu) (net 4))
 (segment (start 146.812 112.1156) (end 147.828 113.1316) (width 0.1524) (layer B.Cu) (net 4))
 (segment (start 147.828 113.1316) (end 147.828 113.284) (width 0.1524) (layer B.Cu) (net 4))
 (segment (start 146.812 106.7435) (end 146.812 112.1156) (width 0.1524) (layer B.Cu) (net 4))
 (segment (start 148.3995 106.3625) (end 147.193 106.3625) (width 0.1524) (layer B.Cu) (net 4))
 (segment (start 147.193 106.3625) (end 146.812 106.7435) (width 0.1524) (layer B.Cu) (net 4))
 (segment (start 148.844 106.807) (end 148.3995 106.3625) (width 0.1524) (layer B.Cu) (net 4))
 (segment (start 149.479 106.172) (end 149.6254 106.172) (width 0.1524) (layer F.Cu) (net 4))
 (segment (start 149.6254 106.172) (end 149.86 105.9374) (width 0.1524) (layer F.Cu) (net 4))
 (segment (start 149.86 105.9374) (end 149.86 105.41) (width 0.1524) (layer F.Cu) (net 4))
 (segment (start 148.844 106.807) (end 149.479 106.172) (width 0.1524) (layer F.Cu) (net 4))
 (segment (start 148.717 106.632018) (end 148.717 106.68) (width 0.1524) (layer F.Cu) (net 4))
 (segment (start 148.717 106.632018) (end 148.784382 106.6994) (width 0.1524) (layer F.Cu) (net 4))
 (segment (start 148.482381 106.397399) (end 148.717 106.632018) (width 0.1524) (layer F.Cu) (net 4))
 (segment (start 148.717 106.68) (end 148.844 106.807) (width 0.1524) (layer F.Cu) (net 4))
 (via (at 148.844 106.807) (size 0.6858) (drill 0.3302) (layers F.Cu B.Cu) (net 4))
 (segment (start 147.9745 106.276) (end 148.095899 106.397399) (width 0.1524) (layer F.Cu) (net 4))
 (segment (start 148.095899 106.397399) (end 148.482381 106.397399) (width 0.1524) (layer F.Cu) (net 4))
 (segment (start 149.86 112.776) (end 149.86 113.2205) (width 0.1524) (layer F.Cu) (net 5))
 (segment (start 149.86 113.2205) (end 150.368 113.7285) (width 0.1524) (layer F.Cu) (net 5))
 (segment (start 149.86 112.776) (end 150.368 113.284) (width 0.1524) (layer F.Cu) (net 5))
 (segment (start 149.86 107.442) (end 149.86 112.776) (width 0.1524) (layer F.Cu) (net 5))
 (segment (start 149.86 107.442) (end 149.86 107.061) (width 0.1524) (layer F.Cu) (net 5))
 (segment (start 147.9745 106.776) (end 147.9745 107.0784) (width 0.1524) (layer F.Cu) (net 5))
 (segment (start 147.9745 107.0784) (end 148.4845 107.5884) (width 0.1524) (layer F.Cu) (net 5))
 (segment (start 148.4845 107.5884) (end 149.3076 107.5884) (width 0.1524) (layer F.Cu) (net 5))
 (segment (start 149.3076 107.5884) (end 149.835 107.061) (width 0.1524) (layer F.Cu) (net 5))
 (segment (start 149.835 107.061) (end 149.86 107.061) (width 0.1524) (layer F.Cu) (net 5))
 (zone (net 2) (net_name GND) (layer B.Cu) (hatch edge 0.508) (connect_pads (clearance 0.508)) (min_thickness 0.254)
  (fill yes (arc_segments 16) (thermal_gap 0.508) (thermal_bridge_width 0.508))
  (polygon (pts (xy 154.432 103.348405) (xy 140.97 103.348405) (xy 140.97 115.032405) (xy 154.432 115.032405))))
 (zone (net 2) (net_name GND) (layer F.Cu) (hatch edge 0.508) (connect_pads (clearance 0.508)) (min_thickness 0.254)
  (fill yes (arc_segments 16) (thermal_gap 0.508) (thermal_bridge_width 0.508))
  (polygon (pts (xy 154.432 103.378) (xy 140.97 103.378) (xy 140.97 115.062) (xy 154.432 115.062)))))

